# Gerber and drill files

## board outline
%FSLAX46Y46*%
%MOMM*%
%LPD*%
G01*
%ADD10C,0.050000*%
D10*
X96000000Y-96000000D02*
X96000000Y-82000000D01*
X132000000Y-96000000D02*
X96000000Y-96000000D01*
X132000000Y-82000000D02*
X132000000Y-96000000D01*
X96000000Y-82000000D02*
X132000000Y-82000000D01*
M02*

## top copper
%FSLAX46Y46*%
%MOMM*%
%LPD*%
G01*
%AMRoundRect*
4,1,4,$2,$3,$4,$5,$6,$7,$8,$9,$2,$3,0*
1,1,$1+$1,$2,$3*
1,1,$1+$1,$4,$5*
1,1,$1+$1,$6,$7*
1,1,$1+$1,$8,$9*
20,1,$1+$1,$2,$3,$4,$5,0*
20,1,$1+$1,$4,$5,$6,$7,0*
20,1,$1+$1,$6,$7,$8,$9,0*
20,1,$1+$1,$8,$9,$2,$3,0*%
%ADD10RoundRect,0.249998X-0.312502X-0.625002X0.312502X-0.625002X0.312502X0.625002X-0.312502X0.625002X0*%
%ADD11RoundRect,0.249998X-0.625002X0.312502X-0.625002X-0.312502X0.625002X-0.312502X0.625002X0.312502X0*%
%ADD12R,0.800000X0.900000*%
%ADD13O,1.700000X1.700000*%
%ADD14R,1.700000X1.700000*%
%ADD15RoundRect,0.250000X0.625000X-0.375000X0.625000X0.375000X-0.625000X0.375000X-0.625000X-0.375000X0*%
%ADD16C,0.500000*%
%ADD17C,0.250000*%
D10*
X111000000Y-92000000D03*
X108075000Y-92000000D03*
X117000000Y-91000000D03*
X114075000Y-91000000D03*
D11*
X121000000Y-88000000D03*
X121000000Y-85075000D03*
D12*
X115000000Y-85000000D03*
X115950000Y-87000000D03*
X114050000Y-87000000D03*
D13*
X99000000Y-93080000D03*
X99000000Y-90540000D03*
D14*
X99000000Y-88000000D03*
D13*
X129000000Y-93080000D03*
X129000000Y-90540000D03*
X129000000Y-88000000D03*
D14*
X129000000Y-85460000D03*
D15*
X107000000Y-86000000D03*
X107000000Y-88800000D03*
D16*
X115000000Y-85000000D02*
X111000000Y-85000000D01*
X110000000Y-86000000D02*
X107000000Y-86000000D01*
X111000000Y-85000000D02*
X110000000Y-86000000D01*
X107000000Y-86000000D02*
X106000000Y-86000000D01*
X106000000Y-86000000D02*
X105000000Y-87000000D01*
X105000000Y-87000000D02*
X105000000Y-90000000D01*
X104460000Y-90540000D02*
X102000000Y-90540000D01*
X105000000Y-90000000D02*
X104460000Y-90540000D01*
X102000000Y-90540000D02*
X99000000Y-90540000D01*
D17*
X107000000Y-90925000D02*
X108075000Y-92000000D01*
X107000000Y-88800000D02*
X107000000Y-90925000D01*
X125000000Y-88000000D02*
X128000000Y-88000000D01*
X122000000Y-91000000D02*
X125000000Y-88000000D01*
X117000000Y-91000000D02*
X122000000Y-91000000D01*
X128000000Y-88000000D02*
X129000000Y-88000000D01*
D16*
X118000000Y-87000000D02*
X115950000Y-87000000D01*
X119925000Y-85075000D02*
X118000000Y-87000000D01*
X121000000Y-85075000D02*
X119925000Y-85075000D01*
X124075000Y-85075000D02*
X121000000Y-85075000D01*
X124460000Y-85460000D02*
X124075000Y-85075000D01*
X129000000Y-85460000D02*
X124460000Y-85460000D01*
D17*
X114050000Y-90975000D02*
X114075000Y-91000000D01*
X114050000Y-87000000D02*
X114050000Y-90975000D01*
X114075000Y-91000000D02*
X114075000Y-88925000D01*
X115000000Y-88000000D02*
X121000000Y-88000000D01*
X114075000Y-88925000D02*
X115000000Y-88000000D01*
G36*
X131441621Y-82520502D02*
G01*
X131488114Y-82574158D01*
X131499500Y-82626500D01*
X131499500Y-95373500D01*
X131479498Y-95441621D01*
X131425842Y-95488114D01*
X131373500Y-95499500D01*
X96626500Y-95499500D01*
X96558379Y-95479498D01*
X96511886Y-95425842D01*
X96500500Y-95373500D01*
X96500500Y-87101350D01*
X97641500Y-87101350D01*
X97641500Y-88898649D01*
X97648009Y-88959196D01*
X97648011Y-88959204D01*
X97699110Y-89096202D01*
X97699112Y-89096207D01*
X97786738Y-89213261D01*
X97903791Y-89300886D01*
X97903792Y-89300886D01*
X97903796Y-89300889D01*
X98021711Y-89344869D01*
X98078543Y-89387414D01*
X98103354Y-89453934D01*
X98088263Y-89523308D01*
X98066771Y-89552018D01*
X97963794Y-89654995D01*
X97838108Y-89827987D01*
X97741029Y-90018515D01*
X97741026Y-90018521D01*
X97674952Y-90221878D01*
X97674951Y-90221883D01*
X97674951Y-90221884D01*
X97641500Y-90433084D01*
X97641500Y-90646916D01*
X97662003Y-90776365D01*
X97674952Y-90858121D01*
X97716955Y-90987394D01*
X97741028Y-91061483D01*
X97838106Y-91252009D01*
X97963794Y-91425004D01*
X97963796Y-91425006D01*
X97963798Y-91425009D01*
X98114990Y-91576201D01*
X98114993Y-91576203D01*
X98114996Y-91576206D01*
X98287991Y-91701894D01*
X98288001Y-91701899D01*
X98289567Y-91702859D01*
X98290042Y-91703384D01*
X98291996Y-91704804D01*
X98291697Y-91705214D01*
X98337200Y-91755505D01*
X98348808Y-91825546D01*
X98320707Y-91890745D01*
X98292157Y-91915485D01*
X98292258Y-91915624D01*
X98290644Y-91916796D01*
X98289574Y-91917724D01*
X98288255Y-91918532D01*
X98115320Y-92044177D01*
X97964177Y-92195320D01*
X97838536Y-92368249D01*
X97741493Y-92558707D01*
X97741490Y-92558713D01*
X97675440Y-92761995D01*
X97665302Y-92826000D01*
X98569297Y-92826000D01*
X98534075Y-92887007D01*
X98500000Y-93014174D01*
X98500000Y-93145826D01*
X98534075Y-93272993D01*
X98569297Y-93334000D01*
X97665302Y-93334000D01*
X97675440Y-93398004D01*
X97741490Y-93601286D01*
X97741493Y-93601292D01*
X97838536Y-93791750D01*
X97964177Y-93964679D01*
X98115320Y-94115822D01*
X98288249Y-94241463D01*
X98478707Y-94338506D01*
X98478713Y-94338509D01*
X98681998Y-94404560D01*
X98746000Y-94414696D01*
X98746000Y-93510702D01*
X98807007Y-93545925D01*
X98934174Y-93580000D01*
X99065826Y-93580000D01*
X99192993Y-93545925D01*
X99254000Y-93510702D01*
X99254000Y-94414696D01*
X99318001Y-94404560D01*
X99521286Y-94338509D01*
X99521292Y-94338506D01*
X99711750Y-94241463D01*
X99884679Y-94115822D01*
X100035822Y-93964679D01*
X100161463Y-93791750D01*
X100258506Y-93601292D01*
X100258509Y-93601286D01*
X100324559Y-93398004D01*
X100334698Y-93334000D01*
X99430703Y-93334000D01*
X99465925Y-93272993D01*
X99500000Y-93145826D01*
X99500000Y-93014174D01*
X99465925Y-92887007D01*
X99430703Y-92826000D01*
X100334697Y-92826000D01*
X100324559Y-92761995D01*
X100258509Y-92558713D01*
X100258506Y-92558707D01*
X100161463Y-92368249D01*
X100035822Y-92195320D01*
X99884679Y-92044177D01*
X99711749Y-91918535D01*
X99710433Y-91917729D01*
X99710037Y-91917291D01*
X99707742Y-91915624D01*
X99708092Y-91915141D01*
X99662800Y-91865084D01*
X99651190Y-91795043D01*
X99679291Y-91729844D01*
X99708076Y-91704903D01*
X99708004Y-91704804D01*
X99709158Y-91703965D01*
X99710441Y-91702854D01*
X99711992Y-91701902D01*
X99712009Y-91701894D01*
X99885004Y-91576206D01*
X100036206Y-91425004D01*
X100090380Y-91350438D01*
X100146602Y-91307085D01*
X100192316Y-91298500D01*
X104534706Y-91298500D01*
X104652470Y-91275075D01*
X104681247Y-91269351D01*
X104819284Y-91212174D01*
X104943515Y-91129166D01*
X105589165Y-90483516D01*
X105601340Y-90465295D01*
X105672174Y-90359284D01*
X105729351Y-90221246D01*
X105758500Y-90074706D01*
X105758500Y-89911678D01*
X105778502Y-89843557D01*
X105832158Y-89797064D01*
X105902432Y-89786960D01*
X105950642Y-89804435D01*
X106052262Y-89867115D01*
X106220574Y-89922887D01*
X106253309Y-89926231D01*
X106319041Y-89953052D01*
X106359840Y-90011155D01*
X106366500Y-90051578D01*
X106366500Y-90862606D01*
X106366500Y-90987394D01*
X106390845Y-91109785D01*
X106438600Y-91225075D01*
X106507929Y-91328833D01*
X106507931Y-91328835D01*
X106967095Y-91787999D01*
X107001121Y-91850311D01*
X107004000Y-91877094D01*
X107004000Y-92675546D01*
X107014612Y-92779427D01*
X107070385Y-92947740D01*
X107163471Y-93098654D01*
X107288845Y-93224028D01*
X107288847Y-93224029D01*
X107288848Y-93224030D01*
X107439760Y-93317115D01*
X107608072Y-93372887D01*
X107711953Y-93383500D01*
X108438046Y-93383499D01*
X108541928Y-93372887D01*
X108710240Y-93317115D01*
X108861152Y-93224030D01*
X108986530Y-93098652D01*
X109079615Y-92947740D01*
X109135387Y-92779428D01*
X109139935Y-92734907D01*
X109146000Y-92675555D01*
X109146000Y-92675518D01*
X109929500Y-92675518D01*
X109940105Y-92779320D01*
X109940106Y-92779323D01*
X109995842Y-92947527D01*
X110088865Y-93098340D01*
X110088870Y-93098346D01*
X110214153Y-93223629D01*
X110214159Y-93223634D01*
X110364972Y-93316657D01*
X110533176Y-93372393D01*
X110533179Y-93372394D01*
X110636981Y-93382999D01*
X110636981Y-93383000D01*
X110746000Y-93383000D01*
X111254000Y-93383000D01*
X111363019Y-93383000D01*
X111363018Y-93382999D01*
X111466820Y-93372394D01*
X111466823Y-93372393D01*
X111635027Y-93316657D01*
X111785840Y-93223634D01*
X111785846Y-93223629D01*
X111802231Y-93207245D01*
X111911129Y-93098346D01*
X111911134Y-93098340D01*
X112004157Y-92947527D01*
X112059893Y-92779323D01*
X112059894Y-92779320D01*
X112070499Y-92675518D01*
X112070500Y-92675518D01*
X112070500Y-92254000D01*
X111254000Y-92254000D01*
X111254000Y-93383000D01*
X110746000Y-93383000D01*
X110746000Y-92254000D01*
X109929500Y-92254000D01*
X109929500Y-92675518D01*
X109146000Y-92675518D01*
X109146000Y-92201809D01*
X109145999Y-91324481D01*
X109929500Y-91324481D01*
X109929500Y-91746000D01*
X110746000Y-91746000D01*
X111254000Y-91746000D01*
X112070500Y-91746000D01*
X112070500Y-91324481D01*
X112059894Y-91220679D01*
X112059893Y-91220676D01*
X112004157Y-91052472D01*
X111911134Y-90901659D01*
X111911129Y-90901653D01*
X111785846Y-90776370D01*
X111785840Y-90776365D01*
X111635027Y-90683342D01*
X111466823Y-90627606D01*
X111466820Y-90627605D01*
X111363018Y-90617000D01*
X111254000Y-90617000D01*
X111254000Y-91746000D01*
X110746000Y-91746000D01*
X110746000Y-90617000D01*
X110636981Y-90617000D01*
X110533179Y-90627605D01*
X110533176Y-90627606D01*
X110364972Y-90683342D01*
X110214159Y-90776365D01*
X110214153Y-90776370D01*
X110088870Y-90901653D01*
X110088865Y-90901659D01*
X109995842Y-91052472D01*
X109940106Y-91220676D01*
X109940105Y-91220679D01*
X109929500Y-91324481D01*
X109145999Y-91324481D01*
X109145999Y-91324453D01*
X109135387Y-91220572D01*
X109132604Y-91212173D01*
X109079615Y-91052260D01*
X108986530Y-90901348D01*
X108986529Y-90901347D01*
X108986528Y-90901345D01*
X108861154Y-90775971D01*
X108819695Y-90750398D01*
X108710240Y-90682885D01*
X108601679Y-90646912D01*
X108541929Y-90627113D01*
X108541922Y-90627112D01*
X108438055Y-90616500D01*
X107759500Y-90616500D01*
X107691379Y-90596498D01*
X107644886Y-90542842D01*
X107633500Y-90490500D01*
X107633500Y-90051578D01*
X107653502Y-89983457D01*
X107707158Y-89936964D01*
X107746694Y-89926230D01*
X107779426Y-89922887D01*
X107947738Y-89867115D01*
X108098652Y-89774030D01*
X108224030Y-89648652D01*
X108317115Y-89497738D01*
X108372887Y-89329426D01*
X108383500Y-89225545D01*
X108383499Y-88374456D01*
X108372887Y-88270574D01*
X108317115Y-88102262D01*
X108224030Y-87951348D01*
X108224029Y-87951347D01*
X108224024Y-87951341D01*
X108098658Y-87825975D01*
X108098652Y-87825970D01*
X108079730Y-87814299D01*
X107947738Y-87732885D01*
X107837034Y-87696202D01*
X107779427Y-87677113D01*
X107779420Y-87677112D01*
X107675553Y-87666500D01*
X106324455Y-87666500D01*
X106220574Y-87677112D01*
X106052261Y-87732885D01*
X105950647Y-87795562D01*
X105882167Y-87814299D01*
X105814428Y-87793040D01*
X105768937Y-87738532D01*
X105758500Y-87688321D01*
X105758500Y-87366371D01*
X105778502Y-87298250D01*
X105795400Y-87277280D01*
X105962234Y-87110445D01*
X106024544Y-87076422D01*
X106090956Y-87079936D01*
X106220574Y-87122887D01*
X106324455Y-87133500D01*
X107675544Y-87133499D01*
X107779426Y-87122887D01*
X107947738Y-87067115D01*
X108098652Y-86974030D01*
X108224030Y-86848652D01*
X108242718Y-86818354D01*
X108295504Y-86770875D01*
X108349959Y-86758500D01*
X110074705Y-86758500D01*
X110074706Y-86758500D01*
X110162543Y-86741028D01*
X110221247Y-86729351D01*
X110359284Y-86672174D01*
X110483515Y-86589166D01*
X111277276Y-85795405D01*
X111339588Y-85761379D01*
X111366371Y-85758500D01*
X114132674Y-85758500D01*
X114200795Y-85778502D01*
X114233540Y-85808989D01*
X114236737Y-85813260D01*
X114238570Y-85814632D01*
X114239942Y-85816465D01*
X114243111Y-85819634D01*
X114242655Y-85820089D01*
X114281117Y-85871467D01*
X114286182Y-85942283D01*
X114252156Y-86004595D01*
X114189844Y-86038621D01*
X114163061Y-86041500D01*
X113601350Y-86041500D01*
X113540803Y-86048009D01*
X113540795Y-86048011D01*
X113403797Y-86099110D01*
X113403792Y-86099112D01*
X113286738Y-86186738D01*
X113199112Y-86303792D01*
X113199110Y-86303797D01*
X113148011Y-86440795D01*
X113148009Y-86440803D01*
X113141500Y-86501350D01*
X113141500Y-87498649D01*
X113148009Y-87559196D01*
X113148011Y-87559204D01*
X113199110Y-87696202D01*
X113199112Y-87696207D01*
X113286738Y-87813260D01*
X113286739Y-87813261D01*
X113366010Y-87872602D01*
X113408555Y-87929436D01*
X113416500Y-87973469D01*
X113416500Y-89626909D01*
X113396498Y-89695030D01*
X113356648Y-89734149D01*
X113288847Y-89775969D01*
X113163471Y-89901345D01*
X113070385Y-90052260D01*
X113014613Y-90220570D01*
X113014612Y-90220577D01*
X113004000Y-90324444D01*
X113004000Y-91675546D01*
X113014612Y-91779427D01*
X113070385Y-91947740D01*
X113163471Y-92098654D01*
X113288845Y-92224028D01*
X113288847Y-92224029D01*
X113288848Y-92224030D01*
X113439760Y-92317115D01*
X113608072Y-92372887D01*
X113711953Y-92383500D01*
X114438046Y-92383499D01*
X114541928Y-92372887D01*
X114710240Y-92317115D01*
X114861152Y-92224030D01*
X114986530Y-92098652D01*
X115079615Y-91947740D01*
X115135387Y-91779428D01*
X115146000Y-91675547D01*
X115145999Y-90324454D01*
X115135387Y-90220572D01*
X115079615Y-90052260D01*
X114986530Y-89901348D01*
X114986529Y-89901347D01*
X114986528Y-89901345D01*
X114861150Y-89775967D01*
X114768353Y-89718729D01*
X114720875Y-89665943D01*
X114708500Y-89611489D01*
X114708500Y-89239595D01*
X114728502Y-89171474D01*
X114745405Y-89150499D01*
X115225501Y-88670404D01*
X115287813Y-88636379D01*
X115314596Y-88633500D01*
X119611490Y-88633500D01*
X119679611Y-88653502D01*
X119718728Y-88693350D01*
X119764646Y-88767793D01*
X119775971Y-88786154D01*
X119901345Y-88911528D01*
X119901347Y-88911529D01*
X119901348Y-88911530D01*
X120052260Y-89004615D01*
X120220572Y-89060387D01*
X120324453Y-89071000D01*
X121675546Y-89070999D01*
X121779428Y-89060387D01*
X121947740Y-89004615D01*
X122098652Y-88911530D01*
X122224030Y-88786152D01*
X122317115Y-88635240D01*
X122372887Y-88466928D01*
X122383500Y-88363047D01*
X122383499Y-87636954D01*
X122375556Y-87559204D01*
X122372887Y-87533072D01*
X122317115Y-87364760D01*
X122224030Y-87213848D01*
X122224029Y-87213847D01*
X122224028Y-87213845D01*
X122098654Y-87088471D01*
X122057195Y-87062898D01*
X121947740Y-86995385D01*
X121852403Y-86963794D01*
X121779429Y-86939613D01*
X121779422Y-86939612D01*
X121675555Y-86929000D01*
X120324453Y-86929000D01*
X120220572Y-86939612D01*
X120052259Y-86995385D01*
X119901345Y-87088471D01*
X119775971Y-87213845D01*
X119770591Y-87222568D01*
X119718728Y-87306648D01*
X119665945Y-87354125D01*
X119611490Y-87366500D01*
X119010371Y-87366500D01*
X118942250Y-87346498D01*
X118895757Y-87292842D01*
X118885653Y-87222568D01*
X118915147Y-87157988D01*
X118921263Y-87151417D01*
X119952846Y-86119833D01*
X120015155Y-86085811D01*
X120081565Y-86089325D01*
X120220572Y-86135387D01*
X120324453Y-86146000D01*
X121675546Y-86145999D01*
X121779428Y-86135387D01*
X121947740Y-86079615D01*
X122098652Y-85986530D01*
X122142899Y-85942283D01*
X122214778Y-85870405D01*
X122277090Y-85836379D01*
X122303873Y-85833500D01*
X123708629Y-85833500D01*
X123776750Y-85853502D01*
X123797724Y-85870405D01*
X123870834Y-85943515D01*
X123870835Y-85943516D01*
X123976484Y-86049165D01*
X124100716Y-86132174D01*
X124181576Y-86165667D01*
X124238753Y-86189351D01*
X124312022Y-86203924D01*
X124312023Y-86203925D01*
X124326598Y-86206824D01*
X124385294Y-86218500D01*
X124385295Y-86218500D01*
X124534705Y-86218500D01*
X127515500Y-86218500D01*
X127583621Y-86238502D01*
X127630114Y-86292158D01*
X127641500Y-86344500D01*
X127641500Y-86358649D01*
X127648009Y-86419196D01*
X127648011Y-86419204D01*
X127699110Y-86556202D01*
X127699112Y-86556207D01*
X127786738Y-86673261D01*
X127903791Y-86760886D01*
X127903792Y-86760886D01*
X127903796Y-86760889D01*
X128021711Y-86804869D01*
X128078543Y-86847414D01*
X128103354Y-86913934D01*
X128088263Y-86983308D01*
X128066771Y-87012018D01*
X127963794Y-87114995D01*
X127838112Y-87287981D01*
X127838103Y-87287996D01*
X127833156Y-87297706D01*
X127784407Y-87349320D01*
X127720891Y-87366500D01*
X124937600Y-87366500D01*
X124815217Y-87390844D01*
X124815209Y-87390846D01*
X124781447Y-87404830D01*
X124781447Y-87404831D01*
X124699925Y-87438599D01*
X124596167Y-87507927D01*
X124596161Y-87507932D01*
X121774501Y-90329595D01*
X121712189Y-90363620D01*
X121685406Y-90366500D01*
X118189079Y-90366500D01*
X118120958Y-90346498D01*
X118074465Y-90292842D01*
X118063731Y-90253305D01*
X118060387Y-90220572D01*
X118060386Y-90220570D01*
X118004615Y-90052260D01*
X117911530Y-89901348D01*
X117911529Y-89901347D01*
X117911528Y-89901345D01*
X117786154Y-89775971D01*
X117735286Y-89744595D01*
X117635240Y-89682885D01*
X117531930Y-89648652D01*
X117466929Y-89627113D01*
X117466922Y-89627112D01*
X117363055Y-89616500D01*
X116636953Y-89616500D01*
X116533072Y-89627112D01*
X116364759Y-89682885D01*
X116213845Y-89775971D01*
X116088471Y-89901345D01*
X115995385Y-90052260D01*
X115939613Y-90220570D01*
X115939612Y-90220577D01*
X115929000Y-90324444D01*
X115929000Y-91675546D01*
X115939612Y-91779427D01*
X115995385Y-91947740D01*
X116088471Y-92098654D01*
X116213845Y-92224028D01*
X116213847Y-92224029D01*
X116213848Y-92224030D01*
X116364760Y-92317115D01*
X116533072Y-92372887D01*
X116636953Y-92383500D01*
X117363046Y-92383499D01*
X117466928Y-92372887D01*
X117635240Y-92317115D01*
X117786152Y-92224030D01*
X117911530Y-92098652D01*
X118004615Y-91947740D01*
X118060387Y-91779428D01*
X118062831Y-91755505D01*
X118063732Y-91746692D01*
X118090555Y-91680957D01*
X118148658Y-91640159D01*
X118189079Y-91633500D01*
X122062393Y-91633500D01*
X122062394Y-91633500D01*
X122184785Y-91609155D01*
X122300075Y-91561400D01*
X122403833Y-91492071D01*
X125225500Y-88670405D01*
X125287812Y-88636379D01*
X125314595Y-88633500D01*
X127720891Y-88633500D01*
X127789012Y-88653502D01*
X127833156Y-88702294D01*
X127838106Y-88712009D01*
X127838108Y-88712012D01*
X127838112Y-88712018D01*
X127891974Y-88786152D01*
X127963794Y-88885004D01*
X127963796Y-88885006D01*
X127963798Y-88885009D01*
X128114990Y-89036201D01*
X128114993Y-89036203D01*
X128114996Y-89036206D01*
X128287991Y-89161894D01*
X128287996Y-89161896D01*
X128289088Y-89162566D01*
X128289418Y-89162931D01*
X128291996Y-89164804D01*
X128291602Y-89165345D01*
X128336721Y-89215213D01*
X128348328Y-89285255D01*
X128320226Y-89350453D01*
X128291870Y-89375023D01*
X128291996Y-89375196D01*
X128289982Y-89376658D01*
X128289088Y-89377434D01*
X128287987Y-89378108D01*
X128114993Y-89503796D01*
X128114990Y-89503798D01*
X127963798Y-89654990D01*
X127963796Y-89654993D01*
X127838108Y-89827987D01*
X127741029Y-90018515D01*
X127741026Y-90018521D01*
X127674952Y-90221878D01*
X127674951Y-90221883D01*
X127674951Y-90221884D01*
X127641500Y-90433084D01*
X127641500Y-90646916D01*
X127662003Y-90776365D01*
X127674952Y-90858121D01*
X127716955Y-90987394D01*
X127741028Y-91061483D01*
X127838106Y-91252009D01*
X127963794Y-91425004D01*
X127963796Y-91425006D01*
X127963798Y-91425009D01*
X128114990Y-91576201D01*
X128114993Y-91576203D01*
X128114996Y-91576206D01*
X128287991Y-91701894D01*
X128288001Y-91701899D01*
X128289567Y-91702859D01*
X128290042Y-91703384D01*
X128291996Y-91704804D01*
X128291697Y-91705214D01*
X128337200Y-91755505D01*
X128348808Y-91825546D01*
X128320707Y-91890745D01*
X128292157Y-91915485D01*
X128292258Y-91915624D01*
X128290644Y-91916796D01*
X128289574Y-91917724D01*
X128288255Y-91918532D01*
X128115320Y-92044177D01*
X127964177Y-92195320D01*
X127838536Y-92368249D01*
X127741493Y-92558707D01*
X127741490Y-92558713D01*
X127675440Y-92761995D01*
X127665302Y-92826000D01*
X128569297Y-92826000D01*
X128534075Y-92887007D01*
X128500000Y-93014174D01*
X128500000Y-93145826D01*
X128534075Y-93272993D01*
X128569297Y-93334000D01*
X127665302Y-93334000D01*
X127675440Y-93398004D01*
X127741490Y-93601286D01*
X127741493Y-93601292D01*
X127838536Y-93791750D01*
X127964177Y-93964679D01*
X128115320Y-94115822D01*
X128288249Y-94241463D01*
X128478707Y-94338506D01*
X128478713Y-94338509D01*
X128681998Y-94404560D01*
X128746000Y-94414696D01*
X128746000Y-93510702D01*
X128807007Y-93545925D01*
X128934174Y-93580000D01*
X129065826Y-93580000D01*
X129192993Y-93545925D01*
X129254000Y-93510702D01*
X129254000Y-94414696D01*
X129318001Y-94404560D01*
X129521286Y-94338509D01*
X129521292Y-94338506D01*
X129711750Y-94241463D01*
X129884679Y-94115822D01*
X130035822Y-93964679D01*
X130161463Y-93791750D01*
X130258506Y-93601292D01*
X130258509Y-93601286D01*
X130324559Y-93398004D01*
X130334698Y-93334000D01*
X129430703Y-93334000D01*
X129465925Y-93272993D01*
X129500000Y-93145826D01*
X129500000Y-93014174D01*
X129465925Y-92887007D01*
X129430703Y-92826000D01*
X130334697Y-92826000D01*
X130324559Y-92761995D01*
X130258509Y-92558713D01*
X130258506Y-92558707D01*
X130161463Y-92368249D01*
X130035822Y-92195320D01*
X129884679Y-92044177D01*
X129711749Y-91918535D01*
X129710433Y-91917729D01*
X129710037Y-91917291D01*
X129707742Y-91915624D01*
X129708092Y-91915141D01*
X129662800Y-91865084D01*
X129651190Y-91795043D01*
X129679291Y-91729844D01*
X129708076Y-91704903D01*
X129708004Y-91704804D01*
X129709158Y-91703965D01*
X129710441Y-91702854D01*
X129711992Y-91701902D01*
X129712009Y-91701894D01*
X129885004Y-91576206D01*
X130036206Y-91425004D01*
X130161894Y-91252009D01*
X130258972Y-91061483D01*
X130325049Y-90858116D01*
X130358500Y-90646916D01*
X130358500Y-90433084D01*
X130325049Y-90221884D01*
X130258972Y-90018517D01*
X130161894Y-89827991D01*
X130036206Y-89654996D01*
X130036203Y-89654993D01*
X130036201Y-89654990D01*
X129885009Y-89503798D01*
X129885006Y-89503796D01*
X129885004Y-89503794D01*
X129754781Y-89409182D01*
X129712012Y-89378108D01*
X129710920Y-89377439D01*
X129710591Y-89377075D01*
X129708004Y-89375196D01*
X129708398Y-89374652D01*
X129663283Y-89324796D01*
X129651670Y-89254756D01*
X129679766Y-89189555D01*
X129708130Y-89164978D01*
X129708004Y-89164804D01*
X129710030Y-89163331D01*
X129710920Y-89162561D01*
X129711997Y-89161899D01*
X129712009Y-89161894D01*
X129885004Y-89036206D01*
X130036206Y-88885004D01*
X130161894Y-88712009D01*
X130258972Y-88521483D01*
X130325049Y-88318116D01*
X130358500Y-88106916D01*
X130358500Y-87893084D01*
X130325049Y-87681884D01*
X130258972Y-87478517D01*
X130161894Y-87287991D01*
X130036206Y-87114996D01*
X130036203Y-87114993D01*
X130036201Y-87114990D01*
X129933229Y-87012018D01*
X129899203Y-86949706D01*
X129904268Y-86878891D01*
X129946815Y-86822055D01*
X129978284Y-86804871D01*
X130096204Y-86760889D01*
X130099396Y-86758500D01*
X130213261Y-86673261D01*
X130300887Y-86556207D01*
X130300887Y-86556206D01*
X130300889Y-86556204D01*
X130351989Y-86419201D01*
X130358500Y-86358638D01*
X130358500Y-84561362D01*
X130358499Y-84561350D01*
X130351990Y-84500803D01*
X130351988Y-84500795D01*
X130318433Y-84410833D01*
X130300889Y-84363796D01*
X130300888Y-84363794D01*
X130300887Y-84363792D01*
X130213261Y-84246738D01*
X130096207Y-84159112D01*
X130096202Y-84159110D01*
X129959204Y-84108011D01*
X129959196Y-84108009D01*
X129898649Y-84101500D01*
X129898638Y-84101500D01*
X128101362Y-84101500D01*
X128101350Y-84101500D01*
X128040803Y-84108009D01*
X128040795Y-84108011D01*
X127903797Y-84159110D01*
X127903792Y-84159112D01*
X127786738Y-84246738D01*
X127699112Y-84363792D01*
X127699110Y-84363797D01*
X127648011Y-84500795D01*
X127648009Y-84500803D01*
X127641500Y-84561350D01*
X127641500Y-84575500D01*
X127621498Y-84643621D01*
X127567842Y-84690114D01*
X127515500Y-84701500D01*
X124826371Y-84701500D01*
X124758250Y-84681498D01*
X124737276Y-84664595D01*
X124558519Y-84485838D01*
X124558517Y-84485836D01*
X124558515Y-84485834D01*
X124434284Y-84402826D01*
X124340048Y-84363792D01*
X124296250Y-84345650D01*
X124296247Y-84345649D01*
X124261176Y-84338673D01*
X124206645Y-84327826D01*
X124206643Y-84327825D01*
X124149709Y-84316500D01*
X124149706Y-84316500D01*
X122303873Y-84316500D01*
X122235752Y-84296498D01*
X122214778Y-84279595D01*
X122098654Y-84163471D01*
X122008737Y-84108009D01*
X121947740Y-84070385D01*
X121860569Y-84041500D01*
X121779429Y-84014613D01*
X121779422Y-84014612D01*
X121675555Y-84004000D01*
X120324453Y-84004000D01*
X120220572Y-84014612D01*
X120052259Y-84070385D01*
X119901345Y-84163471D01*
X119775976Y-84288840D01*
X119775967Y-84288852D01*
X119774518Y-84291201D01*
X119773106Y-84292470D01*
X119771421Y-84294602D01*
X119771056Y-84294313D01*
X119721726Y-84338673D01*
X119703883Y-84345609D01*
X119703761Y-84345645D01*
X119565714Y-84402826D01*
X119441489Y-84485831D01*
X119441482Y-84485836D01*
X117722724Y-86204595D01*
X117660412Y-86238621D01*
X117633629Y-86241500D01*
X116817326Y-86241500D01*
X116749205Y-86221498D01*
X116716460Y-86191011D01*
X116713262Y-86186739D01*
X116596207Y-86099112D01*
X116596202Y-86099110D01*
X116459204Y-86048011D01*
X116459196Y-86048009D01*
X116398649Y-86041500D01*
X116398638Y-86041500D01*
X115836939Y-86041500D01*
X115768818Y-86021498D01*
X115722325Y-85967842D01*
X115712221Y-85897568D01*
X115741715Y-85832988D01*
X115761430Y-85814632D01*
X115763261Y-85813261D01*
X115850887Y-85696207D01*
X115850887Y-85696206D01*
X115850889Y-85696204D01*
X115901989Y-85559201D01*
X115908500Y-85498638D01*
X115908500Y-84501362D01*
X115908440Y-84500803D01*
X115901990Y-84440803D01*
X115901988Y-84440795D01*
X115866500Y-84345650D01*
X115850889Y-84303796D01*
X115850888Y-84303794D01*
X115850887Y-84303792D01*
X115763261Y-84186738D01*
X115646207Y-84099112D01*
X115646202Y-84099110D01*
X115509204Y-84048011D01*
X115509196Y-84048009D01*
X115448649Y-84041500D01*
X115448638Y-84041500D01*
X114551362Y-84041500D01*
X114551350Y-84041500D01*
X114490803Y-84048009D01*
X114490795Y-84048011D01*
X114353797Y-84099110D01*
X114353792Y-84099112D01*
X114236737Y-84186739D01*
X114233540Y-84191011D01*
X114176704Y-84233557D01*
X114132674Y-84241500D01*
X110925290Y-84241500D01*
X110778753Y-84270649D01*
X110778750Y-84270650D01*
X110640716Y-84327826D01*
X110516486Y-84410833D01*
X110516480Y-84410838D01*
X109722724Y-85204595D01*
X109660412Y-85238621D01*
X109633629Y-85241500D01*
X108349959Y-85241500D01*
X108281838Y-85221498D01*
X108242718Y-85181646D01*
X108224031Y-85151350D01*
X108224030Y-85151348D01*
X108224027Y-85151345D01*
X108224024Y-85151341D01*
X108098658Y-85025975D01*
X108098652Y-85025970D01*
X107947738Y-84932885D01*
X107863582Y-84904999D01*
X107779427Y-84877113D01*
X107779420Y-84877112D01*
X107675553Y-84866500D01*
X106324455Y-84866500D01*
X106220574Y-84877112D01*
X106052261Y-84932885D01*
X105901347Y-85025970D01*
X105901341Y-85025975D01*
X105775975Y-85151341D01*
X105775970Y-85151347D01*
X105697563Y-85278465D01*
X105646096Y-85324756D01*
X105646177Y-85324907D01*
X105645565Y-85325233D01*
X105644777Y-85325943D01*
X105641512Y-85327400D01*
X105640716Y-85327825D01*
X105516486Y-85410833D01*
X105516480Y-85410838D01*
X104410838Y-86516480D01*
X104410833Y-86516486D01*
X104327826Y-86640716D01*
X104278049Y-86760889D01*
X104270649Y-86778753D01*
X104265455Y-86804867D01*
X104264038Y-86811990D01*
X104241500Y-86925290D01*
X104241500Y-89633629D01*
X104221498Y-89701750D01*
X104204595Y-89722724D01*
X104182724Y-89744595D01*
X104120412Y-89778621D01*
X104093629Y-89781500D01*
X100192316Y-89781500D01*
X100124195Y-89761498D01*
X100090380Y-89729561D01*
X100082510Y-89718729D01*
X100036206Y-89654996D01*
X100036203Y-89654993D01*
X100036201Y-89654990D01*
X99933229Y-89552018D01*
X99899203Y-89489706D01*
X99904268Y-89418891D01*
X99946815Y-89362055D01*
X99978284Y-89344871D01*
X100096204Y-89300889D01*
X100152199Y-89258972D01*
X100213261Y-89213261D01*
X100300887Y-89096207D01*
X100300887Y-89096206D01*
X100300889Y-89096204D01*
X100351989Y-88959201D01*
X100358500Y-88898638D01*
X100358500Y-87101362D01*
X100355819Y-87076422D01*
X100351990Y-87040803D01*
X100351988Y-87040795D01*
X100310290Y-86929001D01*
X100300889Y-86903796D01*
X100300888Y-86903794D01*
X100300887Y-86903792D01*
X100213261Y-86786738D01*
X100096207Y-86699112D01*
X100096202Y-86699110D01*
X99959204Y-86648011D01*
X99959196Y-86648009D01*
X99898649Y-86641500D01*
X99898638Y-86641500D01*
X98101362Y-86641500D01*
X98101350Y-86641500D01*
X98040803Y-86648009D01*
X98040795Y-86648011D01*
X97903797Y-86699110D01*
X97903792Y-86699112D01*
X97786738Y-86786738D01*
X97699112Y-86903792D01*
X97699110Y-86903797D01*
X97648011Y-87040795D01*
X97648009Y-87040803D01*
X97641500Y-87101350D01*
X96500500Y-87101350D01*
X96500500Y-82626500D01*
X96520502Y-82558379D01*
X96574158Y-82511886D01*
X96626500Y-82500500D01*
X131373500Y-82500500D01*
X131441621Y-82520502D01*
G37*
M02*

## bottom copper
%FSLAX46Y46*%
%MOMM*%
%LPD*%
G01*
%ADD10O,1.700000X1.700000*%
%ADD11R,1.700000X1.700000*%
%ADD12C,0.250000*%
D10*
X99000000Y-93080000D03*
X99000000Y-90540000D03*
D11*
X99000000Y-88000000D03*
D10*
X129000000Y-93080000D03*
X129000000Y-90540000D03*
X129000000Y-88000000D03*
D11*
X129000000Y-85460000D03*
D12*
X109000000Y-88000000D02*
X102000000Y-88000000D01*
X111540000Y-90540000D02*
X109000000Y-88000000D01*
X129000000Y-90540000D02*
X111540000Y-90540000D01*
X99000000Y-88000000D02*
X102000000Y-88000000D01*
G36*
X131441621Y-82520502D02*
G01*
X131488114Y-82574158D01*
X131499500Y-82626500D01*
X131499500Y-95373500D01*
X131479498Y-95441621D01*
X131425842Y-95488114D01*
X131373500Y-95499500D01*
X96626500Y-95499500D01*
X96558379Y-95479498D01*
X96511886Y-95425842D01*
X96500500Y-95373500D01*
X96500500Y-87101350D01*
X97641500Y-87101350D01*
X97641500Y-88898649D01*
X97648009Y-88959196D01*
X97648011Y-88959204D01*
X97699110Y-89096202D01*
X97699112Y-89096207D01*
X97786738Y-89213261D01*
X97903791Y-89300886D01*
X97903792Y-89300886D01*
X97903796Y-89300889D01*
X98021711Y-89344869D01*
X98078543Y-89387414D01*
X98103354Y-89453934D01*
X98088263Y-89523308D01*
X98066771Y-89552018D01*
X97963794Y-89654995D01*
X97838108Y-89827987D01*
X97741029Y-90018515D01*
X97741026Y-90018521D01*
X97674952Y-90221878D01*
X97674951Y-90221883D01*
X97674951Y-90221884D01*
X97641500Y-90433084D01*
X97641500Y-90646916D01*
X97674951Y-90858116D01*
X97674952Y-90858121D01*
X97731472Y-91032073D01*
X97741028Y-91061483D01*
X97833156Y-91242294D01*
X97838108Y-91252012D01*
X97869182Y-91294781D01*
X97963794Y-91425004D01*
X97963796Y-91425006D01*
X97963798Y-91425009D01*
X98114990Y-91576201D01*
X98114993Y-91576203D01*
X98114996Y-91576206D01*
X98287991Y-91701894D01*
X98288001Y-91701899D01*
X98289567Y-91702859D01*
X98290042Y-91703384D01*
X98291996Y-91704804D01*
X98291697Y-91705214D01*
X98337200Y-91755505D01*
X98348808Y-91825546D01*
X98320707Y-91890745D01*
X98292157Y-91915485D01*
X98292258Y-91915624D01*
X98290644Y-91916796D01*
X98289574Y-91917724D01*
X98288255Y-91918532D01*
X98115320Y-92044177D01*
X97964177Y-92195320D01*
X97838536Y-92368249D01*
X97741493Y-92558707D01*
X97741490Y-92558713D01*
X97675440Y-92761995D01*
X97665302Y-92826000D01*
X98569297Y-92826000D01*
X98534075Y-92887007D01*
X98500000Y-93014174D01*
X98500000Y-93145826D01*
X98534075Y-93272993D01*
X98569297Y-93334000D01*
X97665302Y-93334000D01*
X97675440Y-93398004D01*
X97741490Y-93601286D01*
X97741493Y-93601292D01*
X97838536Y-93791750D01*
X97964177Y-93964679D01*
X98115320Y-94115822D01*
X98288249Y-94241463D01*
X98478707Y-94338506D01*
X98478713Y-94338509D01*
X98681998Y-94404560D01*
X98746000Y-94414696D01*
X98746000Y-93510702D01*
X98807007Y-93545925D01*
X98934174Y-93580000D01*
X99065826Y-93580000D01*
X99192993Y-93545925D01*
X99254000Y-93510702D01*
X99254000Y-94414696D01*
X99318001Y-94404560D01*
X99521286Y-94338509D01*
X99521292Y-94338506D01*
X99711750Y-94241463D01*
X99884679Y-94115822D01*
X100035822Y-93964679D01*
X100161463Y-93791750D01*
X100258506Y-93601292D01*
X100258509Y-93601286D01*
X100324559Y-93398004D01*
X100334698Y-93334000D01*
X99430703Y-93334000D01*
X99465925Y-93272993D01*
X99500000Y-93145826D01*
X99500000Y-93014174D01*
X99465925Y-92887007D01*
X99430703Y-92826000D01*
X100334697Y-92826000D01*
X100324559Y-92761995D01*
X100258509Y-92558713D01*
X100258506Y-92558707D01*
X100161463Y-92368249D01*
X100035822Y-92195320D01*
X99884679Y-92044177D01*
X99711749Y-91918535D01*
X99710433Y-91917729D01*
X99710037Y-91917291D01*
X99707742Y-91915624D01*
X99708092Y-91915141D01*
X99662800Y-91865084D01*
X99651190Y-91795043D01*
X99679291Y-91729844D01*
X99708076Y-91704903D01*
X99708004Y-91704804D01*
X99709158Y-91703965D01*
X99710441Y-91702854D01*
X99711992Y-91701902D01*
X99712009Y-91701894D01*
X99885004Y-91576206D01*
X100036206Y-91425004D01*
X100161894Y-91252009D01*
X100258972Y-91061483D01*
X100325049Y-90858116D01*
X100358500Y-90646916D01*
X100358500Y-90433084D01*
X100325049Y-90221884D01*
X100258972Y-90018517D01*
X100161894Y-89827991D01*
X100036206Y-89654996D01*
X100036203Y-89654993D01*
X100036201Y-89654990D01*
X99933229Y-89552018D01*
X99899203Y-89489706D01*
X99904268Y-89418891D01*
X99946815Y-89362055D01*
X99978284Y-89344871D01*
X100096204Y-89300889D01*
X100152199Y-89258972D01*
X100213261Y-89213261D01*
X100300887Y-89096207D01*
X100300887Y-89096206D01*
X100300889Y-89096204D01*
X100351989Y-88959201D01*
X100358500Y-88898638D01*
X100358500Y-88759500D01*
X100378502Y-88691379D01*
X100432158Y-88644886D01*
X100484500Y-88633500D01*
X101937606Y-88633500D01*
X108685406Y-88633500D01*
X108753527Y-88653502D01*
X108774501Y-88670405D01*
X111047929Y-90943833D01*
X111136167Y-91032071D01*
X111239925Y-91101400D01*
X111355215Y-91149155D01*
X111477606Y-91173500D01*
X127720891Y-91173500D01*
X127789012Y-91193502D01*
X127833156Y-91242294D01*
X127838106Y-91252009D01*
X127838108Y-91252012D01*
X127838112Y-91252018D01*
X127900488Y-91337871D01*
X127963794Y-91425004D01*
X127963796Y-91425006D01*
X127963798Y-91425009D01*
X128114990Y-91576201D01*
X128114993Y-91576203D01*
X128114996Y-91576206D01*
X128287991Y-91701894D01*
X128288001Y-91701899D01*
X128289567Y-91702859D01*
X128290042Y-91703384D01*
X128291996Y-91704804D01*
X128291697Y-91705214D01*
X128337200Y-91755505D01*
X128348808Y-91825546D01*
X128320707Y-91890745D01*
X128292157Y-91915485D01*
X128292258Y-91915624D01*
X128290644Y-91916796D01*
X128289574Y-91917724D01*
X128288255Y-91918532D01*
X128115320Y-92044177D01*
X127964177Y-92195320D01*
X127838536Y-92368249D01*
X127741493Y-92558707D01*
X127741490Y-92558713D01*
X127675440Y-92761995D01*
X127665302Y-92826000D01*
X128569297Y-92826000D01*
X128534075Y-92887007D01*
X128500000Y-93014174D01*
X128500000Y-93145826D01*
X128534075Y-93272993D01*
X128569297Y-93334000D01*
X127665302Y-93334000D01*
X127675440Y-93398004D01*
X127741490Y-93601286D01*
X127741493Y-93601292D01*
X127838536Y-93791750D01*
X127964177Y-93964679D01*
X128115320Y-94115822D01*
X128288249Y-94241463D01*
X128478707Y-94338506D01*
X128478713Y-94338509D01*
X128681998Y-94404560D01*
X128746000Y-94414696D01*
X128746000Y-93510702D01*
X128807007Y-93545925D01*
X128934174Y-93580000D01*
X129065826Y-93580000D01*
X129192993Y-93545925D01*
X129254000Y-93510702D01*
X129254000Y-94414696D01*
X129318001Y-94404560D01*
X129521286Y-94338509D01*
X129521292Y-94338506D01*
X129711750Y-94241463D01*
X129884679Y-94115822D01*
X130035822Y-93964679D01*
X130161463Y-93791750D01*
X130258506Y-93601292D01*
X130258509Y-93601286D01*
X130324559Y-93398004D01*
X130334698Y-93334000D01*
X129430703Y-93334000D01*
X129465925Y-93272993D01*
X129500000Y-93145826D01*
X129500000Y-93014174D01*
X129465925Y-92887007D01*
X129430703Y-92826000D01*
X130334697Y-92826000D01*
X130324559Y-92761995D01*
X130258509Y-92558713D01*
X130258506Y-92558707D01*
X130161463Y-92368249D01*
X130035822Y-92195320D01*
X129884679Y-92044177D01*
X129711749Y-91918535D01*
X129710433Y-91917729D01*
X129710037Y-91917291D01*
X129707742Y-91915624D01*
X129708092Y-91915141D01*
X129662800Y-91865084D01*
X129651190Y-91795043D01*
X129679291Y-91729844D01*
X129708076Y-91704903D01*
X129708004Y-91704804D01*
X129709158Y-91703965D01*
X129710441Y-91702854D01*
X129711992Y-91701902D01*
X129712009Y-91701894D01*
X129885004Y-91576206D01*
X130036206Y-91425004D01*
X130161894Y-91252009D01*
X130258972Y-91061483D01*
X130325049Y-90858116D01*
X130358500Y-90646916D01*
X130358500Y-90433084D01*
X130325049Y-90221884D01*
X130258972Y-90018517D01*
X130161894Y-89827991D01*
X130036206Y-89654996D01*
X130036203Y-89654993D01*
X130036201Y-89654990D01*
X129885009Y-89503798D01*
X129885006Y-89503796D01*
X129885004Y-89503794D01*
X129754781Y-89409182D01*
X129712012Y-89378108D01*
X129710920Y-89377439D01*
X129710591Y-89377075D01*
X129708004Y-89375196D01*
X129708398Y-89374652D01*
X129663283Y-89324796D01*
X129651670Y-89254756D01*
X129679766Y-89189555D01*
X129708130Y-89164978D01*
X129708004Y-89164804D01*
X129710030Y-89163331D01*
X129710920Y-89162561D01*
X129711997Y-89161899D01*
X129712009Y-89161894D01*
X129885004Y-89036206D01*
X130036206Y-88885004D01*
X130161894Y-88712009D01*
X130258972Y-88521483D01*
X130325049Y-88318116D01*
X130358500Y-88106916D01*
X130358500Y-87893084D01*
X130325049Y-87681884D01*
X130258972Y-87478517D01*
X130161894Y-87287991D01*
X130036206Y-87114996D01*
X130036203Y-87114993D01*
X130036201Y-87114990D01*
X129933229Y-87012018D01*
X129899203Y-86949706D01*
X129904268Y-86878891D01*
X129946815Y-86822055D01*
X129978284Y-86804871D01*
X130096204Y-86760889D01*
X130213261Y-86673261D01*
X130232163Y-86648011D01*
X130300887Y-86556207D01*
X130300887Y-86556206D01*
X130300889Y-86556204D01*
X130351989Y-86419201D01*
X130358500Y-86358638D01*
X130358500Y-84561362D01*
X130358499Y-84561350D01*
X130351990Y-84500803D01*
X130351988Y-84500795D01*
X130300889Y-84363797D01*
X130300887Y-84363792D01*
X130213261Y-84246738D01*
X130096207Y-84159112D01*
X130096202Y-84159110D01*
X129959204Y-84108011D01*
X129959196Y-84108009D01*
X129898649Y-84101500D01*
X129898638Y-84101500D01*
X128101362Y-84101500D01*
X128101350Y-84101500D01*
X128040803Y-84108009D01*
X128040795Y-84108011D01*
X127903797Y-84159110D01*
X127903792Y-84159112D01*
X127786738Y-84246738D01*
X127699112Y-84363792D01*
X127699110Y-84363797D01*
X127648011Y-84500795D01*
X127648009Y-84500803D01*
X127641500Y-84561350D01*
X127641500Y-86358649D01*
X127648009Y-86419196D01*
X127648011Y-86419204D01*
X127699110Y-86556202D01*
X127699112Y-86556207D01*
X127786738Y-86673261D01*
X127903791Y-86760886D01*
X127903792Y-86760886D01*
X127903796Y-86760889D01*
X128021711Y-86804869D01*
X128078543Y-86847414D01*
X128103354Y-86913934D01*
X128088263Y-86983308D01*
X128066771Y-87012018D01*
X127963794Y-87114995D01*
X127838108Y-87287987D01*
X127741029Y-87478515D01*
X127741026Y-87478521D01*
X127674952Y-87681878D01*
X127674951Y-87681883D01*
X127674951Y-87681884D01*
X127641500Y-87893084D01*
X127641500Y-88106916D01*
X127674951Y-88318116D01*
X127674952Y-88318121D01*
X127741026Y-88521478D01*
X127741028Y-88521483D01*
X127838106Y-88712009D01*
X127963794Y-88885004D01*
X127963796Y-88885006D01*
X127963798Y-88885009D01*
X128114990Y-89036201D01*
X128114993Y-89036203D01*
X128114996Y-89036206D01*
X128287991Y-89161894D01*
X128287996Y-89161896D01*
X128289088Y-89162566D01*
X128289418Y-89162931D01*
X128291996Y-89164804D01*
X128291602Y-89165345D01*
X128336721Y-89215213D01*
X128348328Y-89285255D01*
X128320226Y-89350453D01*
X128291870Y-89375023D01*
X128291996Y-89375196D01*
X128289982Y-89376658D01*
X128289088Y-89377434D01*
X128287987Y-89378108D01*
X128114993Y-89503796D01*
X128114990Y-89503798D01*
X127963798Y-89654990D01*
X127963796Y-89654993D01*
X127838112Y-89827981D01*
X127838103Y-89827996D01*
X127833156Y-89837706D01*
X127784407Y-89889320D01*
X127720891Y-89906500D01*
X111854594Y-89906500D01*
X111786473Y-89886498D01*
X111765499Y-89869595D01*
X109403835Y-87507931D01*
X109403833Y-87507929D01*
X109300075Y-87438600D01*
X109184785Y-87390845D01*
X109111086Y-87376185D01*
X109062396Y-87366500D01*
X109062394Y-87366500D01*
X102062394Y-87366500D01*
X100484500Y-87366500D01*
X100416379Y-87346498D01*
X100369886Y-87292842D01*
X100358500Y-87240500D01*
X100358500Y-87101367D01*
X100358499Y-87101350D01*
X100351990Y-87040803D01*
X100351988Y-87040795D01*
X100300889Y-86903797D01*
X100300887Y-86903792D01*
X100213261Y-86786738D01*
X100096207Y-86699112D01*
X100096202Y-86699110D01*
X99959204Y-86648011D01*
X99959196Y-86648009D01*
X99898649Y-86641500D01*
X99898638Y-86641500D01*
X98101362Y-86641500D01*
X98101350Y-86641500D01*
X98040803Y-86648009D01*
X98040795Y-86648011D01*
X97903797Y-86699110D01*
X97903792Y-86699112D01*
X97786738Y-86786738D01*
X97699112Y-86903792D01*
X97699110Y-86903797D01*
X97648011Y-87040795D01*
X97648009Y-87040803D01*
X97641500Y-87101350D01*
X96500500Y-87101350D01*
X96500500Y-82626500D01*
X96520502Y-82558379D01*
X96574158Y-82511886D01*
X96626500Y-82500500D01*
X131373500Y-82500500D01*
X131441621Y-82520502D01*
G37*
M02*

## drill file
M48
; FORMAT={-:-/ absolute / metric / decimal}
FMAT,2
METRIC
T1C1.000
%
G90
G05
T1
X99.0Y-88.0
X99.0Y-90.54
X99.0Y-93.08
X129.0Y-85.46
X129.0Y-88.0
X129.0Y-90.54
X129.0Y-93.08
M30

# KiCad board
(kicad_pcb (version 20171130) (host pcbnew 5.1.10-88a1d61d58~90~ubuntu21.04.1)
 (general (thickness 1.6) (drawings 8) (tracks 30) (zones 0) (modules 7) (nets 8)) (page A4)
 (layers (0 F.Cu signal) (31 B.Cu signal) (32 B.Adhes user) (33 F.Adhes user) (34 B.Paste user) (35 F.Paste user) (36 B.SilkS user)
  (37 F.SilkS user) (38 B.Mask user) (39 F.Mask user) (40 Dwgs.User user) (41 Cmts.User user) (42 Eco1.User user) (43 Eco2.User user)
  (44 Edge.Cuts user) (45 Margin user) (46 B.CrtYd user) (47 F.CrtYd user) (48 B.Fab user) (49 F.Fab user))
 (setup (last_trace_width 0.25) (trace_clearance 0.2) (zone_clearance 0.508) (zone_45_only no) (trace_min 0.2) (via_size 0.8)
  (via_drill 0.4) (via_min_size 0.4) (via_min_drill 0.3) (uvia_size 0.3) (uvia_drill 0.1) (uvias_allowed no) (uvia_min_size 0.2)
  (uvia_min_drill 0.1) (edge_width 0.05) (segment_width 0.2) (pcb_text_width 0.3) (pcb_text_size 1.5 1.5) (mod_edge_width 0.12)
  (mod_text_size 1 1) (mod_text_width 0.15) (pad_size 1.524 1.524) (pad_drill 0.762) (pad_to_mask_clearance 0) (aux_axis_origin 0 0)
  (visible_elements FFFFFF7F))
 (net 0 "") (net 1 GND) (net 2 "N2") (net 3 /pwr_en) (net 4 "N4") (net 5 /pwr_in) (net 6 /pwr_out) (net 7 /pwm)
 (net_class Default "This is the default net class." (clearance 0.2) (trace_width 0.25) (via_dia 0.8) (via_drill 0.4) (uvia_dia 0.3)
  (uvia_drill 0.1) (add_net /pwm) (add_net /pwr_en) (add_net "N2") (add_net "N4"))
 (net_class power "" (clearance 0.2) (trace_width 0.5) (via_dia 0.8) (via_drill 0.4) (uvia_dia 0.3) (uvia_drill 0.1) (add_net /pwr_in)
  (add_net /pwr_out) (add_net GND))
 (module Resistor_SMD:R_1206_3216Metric (layer F.Cu) (at 109.5375 92)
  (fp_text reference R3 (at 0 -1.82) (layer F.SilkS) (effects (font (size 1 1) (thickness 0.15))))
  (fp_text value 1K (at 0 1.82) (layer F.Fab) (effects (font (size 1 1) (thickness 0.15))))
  (pad 2 smd roundrect (at 1.4625 0) (size 1.125 1.75) (layers F.Cu F.Paste F.Mask) (roundrect_rratio 0.2222204444444444) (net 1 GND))
  (pad 1 smd roundrect (at -1.4625 0) (size 1.125 1.75) (layers F.Cu F.Paste F.Mask) (roundrect_rratio 0.2222204444444444) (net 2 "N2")))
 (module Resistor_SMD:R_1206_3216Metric (layer F.Cu) (at 115.5375 91)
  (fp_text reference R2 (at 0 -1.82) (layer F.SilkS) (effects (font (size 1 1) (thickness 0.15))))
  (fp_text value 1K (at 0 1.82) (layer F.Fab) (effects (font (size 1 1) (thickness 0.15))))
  (pad 2 smd roundrect (at 1.4625 0) (size 1.125 1.75) (layers F.Cu F.Paste F.Mask) (roundrect_rratio 0.2222204444444444) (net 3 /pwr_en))
  (pad 1 smd roundrect (at -1.4625 0) (size 1.125 1.75) (layers F.Cu F.Paste F.Mask) (roundrect_rratio 0.2222204444444444) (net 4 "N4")))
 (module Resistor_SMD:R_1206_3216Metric (layer F.Cu) (at 121 86.5375 270)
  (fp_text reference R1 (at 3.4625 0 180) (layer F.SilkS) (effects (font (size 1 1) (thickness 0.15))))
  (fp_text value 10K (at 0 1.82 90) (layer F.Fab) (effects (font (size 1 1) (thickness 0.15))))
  (pad 2 smd roundrect (at 1.4625 0 270) (size 1.125 1.75) (layers F.Cu F.Paste F.Mask) (roundrect_rratio 0.2222204444444444) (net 4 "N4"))
  (pad 1 smd roundrect (at -1.4625 0 270) (size 1.125 1.75) (layers F.Cu F.Paste F.Mask) (roundrect_rratio 0.2222204444444444)
   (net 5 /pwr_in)))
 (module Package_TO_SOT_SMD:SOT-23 (layer F.Cu) (at 115 86 90)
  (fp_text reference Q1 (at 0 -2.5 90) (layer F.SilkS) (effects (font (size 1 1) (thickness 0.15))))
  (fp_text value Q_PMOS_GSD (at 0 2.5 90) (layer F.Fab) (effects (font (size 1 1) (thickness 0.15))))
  (pad 3 smd rect (at 1 0 90) (size 0.9 0.8) (layers F.Cu F.Paste F.Mask) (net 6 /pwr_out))
  (pad 2 smd rect (at -1 0.95 90) (size 0.9 0.8) (layers F.Cu F.Paste F.Mask) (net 5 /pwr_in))
  (pad 1 smd rect (at -1 -0.95 90) (size 0.9 0.8) (layers F.Cu F.Paste F.Mask) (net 4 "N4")))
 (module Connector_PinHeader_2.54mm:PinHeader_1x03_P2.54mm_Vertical (layer F.Cu) (at 99 88)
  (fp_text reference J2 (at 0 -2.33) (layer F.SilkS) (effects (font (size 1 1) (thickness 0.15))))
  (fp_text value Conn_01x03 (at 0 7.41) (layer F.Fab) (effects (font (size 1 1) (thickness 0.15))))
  (pad 3 thru_hole oval (at 0 5.08) (size 1.7 1.7) (drill 1) (layers *.Cu *.Mask) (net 1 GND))
  (pad 2 thru_hole oval (at 0 2.54) (size 1.7 1.7) (drill 1) (layers *.Cu *.Mask) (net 6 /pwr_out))
  (pad 1 thru_hole rect (at 0 0) (size 1.7 1.7) (drill 1) (layers *.Cu *.Mask) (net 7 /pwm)))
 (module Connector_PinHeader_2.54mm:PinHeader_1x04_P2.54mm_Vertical (layer F.Cu) (at 129 85.46)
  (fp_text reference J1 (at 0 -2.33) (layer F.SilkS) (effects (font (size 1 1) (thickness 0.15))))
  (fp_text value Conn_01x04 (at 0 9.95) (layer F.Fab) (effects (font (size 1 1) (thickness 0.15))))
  (pad 4 thru_hole oval (at 0 7.62) (size 1.7 1.7) (drill 1) (layers *.Cu *.Mask) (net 1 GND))
  (pad 3 thru_hole oval (at 0 5.08) (size 1.7 1.7) (drill 1) (layers *.Cu *.Mask) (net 7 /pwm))
  (pad 2 thru_hole oval (at 0 2.54) (size 1.7 1.7) (drill 1) (layers *.Cu *.Mask) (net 3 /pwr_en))
  (pad 1 thru_hole rect (at 0 0) (size 1.7 1.7) (drill 1) (layers *.Cu *.Mask) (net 5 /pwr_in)))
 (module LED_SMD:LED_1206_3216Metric (layer F.Cu) (at 107 87.4 90)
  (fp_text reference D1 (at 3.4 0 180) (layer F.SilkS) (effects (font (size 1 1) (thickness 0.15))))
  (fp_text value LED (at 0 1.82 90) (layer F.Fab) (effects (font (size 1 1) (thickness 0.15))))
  (pad 2 smd roundrect (at 1.4 0 90) (size 1.25 1.75) (layers F.Cu F.Paste F.Mask) (roundrect_rratio 0.2) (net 6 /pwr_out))
  (pad 1 smd roundrect (at -1.4 0 90) (size 1.25 1.75) (layers F.Cu F.Paste F.Mask) (roundrect_rratio 0.2) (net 2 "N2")))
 (gr_line (start 96 96) (end 96 82) (layer Edge.Cuts) (width 0.05))
 (gr_line (start 132 96) (end 96 96) (layer Edge.Cuts) (width 0.05))
 (gr_line (start 132 82) (end 132 96) (layer Edge.Cuts) (width 0.05))
 (gr_line (start 96 82) (end 132 82) (layer Edge.Cuts) (width 0.05))
 (segment (start 115 85) (end 111 85) (width 0.5) (layer F.Cu) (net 6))
 (segment (start 110 86) (end 107 86) (width 0.5) (layer F.Cu) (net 6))
 (segment (start 111 85) (end 110 86) (width 0.5) (layer F.Cu) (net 6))
 (segment (start 107 86) (end 106 86) (width 0.5) (layer F.Cu) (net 6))
 (segment (start 106 86) (end 105 87) (width 0.5) (layer F.Cu) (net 6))
 (segment (start 105 87) (end 105 90) (width 0.5) (layer F.Cu) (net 6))
 (segment (start 104.46 90.54) (end 102 90.54) (width 0.5) (layer F.Cu) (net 6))
 (segment (start 105 90) (end 104.46 90.54) (width 0.5) (layer F.Cu) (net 6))
 (segment (start 102 90.54) (end 99 90.54) (width 0.5) (layer F.Cu) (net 6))
 (segment (start 107 90.925) (end 108.075 92) (width 0.25) (layer F.Cu) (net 2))
 (segment (start 107 88.8) (end 107 90.925) (width 0.25) (layer F.Cu) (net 2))
 (segment (start 109 88) (end 102 88) (width 0.25) (layer B.Cu) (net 7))
 (segment (start 111.54 90.54) (end 109 88) (width 0.25) (layer B.Cu) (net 7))
 (segment (start 129 90.54) (end 111.54 90.54) (width 0.25) (layer B.Cu) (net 7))
 (segment (start 99 88) (end 102 88) (width 0.25) (layer B.Cu) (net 7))
 (segment (start 125 88) (end 128 88) (width 0.25) (layer F.Cu) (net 3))
 (segment (start 122 91) (end 125 88) (width 0.25) (layer F.Cu) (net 3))
 (segment (start 117 91) (end 122 91) (width 0.25) (layer F.Cu) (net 3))
 (segment (start 128 88) (end 129 88) (width 0.25) (layer F.Cu) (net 3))
 (segment (start 118 87) (end 115.95 87) (width 0.5) (layer F.Cu) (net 5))
 (segment (start 119.925 85.075) (end 118 87) (width 0.5) (layer F.Cu) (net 5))
 (segment (start 121 85.075) (end 119.925 85.075) (width 0.5) (layer F.Cu) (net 5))
 (segment (start 124.075 85.075) (end 121 85.075) (width 0.5) (layer F.Cu) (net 5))
 (segment (start 124.46 85.46) (end 124.075 85.075) (width 0.5) (layer F.Cu) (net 5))
 (segment (start 129 85.46) (end 124.46 85.46) (width 0.5) (layer F.Cu) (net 5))
 (segment (start 114.05 90.975) (end 114.075 91) (width 0.25) (layer F.Cu) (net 4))
 (segment (start 114.05 87) (end 114.05 90.975) (width 0.25) (layer F.Cu) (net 4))
 (segment (start 114.075 91) (end 114.075 88.925) (width 0.25) (layer F.Cu) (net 4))
 (segment (start 115 88) (end 121 88) (width 0.25) (layer F.Cu) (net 4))
 (segment (start 114.075 88.925) (end 115 88) (width 0.25) (layer F.Cu) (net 4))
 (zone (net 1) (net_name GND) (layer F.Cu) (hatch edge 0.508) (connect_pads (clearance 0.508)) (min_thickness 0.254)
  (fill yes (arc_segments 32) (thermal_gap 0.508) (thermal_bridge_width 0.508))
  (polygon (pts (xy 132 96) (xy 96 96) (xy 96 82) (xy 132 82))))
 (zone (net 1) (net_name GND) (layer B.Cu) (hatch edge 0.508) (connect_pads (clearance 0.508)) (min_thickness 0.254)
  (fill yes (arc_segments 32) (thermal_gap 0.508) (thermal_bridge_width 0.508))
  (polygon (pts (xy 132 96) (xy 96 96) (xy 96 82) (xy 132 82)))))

